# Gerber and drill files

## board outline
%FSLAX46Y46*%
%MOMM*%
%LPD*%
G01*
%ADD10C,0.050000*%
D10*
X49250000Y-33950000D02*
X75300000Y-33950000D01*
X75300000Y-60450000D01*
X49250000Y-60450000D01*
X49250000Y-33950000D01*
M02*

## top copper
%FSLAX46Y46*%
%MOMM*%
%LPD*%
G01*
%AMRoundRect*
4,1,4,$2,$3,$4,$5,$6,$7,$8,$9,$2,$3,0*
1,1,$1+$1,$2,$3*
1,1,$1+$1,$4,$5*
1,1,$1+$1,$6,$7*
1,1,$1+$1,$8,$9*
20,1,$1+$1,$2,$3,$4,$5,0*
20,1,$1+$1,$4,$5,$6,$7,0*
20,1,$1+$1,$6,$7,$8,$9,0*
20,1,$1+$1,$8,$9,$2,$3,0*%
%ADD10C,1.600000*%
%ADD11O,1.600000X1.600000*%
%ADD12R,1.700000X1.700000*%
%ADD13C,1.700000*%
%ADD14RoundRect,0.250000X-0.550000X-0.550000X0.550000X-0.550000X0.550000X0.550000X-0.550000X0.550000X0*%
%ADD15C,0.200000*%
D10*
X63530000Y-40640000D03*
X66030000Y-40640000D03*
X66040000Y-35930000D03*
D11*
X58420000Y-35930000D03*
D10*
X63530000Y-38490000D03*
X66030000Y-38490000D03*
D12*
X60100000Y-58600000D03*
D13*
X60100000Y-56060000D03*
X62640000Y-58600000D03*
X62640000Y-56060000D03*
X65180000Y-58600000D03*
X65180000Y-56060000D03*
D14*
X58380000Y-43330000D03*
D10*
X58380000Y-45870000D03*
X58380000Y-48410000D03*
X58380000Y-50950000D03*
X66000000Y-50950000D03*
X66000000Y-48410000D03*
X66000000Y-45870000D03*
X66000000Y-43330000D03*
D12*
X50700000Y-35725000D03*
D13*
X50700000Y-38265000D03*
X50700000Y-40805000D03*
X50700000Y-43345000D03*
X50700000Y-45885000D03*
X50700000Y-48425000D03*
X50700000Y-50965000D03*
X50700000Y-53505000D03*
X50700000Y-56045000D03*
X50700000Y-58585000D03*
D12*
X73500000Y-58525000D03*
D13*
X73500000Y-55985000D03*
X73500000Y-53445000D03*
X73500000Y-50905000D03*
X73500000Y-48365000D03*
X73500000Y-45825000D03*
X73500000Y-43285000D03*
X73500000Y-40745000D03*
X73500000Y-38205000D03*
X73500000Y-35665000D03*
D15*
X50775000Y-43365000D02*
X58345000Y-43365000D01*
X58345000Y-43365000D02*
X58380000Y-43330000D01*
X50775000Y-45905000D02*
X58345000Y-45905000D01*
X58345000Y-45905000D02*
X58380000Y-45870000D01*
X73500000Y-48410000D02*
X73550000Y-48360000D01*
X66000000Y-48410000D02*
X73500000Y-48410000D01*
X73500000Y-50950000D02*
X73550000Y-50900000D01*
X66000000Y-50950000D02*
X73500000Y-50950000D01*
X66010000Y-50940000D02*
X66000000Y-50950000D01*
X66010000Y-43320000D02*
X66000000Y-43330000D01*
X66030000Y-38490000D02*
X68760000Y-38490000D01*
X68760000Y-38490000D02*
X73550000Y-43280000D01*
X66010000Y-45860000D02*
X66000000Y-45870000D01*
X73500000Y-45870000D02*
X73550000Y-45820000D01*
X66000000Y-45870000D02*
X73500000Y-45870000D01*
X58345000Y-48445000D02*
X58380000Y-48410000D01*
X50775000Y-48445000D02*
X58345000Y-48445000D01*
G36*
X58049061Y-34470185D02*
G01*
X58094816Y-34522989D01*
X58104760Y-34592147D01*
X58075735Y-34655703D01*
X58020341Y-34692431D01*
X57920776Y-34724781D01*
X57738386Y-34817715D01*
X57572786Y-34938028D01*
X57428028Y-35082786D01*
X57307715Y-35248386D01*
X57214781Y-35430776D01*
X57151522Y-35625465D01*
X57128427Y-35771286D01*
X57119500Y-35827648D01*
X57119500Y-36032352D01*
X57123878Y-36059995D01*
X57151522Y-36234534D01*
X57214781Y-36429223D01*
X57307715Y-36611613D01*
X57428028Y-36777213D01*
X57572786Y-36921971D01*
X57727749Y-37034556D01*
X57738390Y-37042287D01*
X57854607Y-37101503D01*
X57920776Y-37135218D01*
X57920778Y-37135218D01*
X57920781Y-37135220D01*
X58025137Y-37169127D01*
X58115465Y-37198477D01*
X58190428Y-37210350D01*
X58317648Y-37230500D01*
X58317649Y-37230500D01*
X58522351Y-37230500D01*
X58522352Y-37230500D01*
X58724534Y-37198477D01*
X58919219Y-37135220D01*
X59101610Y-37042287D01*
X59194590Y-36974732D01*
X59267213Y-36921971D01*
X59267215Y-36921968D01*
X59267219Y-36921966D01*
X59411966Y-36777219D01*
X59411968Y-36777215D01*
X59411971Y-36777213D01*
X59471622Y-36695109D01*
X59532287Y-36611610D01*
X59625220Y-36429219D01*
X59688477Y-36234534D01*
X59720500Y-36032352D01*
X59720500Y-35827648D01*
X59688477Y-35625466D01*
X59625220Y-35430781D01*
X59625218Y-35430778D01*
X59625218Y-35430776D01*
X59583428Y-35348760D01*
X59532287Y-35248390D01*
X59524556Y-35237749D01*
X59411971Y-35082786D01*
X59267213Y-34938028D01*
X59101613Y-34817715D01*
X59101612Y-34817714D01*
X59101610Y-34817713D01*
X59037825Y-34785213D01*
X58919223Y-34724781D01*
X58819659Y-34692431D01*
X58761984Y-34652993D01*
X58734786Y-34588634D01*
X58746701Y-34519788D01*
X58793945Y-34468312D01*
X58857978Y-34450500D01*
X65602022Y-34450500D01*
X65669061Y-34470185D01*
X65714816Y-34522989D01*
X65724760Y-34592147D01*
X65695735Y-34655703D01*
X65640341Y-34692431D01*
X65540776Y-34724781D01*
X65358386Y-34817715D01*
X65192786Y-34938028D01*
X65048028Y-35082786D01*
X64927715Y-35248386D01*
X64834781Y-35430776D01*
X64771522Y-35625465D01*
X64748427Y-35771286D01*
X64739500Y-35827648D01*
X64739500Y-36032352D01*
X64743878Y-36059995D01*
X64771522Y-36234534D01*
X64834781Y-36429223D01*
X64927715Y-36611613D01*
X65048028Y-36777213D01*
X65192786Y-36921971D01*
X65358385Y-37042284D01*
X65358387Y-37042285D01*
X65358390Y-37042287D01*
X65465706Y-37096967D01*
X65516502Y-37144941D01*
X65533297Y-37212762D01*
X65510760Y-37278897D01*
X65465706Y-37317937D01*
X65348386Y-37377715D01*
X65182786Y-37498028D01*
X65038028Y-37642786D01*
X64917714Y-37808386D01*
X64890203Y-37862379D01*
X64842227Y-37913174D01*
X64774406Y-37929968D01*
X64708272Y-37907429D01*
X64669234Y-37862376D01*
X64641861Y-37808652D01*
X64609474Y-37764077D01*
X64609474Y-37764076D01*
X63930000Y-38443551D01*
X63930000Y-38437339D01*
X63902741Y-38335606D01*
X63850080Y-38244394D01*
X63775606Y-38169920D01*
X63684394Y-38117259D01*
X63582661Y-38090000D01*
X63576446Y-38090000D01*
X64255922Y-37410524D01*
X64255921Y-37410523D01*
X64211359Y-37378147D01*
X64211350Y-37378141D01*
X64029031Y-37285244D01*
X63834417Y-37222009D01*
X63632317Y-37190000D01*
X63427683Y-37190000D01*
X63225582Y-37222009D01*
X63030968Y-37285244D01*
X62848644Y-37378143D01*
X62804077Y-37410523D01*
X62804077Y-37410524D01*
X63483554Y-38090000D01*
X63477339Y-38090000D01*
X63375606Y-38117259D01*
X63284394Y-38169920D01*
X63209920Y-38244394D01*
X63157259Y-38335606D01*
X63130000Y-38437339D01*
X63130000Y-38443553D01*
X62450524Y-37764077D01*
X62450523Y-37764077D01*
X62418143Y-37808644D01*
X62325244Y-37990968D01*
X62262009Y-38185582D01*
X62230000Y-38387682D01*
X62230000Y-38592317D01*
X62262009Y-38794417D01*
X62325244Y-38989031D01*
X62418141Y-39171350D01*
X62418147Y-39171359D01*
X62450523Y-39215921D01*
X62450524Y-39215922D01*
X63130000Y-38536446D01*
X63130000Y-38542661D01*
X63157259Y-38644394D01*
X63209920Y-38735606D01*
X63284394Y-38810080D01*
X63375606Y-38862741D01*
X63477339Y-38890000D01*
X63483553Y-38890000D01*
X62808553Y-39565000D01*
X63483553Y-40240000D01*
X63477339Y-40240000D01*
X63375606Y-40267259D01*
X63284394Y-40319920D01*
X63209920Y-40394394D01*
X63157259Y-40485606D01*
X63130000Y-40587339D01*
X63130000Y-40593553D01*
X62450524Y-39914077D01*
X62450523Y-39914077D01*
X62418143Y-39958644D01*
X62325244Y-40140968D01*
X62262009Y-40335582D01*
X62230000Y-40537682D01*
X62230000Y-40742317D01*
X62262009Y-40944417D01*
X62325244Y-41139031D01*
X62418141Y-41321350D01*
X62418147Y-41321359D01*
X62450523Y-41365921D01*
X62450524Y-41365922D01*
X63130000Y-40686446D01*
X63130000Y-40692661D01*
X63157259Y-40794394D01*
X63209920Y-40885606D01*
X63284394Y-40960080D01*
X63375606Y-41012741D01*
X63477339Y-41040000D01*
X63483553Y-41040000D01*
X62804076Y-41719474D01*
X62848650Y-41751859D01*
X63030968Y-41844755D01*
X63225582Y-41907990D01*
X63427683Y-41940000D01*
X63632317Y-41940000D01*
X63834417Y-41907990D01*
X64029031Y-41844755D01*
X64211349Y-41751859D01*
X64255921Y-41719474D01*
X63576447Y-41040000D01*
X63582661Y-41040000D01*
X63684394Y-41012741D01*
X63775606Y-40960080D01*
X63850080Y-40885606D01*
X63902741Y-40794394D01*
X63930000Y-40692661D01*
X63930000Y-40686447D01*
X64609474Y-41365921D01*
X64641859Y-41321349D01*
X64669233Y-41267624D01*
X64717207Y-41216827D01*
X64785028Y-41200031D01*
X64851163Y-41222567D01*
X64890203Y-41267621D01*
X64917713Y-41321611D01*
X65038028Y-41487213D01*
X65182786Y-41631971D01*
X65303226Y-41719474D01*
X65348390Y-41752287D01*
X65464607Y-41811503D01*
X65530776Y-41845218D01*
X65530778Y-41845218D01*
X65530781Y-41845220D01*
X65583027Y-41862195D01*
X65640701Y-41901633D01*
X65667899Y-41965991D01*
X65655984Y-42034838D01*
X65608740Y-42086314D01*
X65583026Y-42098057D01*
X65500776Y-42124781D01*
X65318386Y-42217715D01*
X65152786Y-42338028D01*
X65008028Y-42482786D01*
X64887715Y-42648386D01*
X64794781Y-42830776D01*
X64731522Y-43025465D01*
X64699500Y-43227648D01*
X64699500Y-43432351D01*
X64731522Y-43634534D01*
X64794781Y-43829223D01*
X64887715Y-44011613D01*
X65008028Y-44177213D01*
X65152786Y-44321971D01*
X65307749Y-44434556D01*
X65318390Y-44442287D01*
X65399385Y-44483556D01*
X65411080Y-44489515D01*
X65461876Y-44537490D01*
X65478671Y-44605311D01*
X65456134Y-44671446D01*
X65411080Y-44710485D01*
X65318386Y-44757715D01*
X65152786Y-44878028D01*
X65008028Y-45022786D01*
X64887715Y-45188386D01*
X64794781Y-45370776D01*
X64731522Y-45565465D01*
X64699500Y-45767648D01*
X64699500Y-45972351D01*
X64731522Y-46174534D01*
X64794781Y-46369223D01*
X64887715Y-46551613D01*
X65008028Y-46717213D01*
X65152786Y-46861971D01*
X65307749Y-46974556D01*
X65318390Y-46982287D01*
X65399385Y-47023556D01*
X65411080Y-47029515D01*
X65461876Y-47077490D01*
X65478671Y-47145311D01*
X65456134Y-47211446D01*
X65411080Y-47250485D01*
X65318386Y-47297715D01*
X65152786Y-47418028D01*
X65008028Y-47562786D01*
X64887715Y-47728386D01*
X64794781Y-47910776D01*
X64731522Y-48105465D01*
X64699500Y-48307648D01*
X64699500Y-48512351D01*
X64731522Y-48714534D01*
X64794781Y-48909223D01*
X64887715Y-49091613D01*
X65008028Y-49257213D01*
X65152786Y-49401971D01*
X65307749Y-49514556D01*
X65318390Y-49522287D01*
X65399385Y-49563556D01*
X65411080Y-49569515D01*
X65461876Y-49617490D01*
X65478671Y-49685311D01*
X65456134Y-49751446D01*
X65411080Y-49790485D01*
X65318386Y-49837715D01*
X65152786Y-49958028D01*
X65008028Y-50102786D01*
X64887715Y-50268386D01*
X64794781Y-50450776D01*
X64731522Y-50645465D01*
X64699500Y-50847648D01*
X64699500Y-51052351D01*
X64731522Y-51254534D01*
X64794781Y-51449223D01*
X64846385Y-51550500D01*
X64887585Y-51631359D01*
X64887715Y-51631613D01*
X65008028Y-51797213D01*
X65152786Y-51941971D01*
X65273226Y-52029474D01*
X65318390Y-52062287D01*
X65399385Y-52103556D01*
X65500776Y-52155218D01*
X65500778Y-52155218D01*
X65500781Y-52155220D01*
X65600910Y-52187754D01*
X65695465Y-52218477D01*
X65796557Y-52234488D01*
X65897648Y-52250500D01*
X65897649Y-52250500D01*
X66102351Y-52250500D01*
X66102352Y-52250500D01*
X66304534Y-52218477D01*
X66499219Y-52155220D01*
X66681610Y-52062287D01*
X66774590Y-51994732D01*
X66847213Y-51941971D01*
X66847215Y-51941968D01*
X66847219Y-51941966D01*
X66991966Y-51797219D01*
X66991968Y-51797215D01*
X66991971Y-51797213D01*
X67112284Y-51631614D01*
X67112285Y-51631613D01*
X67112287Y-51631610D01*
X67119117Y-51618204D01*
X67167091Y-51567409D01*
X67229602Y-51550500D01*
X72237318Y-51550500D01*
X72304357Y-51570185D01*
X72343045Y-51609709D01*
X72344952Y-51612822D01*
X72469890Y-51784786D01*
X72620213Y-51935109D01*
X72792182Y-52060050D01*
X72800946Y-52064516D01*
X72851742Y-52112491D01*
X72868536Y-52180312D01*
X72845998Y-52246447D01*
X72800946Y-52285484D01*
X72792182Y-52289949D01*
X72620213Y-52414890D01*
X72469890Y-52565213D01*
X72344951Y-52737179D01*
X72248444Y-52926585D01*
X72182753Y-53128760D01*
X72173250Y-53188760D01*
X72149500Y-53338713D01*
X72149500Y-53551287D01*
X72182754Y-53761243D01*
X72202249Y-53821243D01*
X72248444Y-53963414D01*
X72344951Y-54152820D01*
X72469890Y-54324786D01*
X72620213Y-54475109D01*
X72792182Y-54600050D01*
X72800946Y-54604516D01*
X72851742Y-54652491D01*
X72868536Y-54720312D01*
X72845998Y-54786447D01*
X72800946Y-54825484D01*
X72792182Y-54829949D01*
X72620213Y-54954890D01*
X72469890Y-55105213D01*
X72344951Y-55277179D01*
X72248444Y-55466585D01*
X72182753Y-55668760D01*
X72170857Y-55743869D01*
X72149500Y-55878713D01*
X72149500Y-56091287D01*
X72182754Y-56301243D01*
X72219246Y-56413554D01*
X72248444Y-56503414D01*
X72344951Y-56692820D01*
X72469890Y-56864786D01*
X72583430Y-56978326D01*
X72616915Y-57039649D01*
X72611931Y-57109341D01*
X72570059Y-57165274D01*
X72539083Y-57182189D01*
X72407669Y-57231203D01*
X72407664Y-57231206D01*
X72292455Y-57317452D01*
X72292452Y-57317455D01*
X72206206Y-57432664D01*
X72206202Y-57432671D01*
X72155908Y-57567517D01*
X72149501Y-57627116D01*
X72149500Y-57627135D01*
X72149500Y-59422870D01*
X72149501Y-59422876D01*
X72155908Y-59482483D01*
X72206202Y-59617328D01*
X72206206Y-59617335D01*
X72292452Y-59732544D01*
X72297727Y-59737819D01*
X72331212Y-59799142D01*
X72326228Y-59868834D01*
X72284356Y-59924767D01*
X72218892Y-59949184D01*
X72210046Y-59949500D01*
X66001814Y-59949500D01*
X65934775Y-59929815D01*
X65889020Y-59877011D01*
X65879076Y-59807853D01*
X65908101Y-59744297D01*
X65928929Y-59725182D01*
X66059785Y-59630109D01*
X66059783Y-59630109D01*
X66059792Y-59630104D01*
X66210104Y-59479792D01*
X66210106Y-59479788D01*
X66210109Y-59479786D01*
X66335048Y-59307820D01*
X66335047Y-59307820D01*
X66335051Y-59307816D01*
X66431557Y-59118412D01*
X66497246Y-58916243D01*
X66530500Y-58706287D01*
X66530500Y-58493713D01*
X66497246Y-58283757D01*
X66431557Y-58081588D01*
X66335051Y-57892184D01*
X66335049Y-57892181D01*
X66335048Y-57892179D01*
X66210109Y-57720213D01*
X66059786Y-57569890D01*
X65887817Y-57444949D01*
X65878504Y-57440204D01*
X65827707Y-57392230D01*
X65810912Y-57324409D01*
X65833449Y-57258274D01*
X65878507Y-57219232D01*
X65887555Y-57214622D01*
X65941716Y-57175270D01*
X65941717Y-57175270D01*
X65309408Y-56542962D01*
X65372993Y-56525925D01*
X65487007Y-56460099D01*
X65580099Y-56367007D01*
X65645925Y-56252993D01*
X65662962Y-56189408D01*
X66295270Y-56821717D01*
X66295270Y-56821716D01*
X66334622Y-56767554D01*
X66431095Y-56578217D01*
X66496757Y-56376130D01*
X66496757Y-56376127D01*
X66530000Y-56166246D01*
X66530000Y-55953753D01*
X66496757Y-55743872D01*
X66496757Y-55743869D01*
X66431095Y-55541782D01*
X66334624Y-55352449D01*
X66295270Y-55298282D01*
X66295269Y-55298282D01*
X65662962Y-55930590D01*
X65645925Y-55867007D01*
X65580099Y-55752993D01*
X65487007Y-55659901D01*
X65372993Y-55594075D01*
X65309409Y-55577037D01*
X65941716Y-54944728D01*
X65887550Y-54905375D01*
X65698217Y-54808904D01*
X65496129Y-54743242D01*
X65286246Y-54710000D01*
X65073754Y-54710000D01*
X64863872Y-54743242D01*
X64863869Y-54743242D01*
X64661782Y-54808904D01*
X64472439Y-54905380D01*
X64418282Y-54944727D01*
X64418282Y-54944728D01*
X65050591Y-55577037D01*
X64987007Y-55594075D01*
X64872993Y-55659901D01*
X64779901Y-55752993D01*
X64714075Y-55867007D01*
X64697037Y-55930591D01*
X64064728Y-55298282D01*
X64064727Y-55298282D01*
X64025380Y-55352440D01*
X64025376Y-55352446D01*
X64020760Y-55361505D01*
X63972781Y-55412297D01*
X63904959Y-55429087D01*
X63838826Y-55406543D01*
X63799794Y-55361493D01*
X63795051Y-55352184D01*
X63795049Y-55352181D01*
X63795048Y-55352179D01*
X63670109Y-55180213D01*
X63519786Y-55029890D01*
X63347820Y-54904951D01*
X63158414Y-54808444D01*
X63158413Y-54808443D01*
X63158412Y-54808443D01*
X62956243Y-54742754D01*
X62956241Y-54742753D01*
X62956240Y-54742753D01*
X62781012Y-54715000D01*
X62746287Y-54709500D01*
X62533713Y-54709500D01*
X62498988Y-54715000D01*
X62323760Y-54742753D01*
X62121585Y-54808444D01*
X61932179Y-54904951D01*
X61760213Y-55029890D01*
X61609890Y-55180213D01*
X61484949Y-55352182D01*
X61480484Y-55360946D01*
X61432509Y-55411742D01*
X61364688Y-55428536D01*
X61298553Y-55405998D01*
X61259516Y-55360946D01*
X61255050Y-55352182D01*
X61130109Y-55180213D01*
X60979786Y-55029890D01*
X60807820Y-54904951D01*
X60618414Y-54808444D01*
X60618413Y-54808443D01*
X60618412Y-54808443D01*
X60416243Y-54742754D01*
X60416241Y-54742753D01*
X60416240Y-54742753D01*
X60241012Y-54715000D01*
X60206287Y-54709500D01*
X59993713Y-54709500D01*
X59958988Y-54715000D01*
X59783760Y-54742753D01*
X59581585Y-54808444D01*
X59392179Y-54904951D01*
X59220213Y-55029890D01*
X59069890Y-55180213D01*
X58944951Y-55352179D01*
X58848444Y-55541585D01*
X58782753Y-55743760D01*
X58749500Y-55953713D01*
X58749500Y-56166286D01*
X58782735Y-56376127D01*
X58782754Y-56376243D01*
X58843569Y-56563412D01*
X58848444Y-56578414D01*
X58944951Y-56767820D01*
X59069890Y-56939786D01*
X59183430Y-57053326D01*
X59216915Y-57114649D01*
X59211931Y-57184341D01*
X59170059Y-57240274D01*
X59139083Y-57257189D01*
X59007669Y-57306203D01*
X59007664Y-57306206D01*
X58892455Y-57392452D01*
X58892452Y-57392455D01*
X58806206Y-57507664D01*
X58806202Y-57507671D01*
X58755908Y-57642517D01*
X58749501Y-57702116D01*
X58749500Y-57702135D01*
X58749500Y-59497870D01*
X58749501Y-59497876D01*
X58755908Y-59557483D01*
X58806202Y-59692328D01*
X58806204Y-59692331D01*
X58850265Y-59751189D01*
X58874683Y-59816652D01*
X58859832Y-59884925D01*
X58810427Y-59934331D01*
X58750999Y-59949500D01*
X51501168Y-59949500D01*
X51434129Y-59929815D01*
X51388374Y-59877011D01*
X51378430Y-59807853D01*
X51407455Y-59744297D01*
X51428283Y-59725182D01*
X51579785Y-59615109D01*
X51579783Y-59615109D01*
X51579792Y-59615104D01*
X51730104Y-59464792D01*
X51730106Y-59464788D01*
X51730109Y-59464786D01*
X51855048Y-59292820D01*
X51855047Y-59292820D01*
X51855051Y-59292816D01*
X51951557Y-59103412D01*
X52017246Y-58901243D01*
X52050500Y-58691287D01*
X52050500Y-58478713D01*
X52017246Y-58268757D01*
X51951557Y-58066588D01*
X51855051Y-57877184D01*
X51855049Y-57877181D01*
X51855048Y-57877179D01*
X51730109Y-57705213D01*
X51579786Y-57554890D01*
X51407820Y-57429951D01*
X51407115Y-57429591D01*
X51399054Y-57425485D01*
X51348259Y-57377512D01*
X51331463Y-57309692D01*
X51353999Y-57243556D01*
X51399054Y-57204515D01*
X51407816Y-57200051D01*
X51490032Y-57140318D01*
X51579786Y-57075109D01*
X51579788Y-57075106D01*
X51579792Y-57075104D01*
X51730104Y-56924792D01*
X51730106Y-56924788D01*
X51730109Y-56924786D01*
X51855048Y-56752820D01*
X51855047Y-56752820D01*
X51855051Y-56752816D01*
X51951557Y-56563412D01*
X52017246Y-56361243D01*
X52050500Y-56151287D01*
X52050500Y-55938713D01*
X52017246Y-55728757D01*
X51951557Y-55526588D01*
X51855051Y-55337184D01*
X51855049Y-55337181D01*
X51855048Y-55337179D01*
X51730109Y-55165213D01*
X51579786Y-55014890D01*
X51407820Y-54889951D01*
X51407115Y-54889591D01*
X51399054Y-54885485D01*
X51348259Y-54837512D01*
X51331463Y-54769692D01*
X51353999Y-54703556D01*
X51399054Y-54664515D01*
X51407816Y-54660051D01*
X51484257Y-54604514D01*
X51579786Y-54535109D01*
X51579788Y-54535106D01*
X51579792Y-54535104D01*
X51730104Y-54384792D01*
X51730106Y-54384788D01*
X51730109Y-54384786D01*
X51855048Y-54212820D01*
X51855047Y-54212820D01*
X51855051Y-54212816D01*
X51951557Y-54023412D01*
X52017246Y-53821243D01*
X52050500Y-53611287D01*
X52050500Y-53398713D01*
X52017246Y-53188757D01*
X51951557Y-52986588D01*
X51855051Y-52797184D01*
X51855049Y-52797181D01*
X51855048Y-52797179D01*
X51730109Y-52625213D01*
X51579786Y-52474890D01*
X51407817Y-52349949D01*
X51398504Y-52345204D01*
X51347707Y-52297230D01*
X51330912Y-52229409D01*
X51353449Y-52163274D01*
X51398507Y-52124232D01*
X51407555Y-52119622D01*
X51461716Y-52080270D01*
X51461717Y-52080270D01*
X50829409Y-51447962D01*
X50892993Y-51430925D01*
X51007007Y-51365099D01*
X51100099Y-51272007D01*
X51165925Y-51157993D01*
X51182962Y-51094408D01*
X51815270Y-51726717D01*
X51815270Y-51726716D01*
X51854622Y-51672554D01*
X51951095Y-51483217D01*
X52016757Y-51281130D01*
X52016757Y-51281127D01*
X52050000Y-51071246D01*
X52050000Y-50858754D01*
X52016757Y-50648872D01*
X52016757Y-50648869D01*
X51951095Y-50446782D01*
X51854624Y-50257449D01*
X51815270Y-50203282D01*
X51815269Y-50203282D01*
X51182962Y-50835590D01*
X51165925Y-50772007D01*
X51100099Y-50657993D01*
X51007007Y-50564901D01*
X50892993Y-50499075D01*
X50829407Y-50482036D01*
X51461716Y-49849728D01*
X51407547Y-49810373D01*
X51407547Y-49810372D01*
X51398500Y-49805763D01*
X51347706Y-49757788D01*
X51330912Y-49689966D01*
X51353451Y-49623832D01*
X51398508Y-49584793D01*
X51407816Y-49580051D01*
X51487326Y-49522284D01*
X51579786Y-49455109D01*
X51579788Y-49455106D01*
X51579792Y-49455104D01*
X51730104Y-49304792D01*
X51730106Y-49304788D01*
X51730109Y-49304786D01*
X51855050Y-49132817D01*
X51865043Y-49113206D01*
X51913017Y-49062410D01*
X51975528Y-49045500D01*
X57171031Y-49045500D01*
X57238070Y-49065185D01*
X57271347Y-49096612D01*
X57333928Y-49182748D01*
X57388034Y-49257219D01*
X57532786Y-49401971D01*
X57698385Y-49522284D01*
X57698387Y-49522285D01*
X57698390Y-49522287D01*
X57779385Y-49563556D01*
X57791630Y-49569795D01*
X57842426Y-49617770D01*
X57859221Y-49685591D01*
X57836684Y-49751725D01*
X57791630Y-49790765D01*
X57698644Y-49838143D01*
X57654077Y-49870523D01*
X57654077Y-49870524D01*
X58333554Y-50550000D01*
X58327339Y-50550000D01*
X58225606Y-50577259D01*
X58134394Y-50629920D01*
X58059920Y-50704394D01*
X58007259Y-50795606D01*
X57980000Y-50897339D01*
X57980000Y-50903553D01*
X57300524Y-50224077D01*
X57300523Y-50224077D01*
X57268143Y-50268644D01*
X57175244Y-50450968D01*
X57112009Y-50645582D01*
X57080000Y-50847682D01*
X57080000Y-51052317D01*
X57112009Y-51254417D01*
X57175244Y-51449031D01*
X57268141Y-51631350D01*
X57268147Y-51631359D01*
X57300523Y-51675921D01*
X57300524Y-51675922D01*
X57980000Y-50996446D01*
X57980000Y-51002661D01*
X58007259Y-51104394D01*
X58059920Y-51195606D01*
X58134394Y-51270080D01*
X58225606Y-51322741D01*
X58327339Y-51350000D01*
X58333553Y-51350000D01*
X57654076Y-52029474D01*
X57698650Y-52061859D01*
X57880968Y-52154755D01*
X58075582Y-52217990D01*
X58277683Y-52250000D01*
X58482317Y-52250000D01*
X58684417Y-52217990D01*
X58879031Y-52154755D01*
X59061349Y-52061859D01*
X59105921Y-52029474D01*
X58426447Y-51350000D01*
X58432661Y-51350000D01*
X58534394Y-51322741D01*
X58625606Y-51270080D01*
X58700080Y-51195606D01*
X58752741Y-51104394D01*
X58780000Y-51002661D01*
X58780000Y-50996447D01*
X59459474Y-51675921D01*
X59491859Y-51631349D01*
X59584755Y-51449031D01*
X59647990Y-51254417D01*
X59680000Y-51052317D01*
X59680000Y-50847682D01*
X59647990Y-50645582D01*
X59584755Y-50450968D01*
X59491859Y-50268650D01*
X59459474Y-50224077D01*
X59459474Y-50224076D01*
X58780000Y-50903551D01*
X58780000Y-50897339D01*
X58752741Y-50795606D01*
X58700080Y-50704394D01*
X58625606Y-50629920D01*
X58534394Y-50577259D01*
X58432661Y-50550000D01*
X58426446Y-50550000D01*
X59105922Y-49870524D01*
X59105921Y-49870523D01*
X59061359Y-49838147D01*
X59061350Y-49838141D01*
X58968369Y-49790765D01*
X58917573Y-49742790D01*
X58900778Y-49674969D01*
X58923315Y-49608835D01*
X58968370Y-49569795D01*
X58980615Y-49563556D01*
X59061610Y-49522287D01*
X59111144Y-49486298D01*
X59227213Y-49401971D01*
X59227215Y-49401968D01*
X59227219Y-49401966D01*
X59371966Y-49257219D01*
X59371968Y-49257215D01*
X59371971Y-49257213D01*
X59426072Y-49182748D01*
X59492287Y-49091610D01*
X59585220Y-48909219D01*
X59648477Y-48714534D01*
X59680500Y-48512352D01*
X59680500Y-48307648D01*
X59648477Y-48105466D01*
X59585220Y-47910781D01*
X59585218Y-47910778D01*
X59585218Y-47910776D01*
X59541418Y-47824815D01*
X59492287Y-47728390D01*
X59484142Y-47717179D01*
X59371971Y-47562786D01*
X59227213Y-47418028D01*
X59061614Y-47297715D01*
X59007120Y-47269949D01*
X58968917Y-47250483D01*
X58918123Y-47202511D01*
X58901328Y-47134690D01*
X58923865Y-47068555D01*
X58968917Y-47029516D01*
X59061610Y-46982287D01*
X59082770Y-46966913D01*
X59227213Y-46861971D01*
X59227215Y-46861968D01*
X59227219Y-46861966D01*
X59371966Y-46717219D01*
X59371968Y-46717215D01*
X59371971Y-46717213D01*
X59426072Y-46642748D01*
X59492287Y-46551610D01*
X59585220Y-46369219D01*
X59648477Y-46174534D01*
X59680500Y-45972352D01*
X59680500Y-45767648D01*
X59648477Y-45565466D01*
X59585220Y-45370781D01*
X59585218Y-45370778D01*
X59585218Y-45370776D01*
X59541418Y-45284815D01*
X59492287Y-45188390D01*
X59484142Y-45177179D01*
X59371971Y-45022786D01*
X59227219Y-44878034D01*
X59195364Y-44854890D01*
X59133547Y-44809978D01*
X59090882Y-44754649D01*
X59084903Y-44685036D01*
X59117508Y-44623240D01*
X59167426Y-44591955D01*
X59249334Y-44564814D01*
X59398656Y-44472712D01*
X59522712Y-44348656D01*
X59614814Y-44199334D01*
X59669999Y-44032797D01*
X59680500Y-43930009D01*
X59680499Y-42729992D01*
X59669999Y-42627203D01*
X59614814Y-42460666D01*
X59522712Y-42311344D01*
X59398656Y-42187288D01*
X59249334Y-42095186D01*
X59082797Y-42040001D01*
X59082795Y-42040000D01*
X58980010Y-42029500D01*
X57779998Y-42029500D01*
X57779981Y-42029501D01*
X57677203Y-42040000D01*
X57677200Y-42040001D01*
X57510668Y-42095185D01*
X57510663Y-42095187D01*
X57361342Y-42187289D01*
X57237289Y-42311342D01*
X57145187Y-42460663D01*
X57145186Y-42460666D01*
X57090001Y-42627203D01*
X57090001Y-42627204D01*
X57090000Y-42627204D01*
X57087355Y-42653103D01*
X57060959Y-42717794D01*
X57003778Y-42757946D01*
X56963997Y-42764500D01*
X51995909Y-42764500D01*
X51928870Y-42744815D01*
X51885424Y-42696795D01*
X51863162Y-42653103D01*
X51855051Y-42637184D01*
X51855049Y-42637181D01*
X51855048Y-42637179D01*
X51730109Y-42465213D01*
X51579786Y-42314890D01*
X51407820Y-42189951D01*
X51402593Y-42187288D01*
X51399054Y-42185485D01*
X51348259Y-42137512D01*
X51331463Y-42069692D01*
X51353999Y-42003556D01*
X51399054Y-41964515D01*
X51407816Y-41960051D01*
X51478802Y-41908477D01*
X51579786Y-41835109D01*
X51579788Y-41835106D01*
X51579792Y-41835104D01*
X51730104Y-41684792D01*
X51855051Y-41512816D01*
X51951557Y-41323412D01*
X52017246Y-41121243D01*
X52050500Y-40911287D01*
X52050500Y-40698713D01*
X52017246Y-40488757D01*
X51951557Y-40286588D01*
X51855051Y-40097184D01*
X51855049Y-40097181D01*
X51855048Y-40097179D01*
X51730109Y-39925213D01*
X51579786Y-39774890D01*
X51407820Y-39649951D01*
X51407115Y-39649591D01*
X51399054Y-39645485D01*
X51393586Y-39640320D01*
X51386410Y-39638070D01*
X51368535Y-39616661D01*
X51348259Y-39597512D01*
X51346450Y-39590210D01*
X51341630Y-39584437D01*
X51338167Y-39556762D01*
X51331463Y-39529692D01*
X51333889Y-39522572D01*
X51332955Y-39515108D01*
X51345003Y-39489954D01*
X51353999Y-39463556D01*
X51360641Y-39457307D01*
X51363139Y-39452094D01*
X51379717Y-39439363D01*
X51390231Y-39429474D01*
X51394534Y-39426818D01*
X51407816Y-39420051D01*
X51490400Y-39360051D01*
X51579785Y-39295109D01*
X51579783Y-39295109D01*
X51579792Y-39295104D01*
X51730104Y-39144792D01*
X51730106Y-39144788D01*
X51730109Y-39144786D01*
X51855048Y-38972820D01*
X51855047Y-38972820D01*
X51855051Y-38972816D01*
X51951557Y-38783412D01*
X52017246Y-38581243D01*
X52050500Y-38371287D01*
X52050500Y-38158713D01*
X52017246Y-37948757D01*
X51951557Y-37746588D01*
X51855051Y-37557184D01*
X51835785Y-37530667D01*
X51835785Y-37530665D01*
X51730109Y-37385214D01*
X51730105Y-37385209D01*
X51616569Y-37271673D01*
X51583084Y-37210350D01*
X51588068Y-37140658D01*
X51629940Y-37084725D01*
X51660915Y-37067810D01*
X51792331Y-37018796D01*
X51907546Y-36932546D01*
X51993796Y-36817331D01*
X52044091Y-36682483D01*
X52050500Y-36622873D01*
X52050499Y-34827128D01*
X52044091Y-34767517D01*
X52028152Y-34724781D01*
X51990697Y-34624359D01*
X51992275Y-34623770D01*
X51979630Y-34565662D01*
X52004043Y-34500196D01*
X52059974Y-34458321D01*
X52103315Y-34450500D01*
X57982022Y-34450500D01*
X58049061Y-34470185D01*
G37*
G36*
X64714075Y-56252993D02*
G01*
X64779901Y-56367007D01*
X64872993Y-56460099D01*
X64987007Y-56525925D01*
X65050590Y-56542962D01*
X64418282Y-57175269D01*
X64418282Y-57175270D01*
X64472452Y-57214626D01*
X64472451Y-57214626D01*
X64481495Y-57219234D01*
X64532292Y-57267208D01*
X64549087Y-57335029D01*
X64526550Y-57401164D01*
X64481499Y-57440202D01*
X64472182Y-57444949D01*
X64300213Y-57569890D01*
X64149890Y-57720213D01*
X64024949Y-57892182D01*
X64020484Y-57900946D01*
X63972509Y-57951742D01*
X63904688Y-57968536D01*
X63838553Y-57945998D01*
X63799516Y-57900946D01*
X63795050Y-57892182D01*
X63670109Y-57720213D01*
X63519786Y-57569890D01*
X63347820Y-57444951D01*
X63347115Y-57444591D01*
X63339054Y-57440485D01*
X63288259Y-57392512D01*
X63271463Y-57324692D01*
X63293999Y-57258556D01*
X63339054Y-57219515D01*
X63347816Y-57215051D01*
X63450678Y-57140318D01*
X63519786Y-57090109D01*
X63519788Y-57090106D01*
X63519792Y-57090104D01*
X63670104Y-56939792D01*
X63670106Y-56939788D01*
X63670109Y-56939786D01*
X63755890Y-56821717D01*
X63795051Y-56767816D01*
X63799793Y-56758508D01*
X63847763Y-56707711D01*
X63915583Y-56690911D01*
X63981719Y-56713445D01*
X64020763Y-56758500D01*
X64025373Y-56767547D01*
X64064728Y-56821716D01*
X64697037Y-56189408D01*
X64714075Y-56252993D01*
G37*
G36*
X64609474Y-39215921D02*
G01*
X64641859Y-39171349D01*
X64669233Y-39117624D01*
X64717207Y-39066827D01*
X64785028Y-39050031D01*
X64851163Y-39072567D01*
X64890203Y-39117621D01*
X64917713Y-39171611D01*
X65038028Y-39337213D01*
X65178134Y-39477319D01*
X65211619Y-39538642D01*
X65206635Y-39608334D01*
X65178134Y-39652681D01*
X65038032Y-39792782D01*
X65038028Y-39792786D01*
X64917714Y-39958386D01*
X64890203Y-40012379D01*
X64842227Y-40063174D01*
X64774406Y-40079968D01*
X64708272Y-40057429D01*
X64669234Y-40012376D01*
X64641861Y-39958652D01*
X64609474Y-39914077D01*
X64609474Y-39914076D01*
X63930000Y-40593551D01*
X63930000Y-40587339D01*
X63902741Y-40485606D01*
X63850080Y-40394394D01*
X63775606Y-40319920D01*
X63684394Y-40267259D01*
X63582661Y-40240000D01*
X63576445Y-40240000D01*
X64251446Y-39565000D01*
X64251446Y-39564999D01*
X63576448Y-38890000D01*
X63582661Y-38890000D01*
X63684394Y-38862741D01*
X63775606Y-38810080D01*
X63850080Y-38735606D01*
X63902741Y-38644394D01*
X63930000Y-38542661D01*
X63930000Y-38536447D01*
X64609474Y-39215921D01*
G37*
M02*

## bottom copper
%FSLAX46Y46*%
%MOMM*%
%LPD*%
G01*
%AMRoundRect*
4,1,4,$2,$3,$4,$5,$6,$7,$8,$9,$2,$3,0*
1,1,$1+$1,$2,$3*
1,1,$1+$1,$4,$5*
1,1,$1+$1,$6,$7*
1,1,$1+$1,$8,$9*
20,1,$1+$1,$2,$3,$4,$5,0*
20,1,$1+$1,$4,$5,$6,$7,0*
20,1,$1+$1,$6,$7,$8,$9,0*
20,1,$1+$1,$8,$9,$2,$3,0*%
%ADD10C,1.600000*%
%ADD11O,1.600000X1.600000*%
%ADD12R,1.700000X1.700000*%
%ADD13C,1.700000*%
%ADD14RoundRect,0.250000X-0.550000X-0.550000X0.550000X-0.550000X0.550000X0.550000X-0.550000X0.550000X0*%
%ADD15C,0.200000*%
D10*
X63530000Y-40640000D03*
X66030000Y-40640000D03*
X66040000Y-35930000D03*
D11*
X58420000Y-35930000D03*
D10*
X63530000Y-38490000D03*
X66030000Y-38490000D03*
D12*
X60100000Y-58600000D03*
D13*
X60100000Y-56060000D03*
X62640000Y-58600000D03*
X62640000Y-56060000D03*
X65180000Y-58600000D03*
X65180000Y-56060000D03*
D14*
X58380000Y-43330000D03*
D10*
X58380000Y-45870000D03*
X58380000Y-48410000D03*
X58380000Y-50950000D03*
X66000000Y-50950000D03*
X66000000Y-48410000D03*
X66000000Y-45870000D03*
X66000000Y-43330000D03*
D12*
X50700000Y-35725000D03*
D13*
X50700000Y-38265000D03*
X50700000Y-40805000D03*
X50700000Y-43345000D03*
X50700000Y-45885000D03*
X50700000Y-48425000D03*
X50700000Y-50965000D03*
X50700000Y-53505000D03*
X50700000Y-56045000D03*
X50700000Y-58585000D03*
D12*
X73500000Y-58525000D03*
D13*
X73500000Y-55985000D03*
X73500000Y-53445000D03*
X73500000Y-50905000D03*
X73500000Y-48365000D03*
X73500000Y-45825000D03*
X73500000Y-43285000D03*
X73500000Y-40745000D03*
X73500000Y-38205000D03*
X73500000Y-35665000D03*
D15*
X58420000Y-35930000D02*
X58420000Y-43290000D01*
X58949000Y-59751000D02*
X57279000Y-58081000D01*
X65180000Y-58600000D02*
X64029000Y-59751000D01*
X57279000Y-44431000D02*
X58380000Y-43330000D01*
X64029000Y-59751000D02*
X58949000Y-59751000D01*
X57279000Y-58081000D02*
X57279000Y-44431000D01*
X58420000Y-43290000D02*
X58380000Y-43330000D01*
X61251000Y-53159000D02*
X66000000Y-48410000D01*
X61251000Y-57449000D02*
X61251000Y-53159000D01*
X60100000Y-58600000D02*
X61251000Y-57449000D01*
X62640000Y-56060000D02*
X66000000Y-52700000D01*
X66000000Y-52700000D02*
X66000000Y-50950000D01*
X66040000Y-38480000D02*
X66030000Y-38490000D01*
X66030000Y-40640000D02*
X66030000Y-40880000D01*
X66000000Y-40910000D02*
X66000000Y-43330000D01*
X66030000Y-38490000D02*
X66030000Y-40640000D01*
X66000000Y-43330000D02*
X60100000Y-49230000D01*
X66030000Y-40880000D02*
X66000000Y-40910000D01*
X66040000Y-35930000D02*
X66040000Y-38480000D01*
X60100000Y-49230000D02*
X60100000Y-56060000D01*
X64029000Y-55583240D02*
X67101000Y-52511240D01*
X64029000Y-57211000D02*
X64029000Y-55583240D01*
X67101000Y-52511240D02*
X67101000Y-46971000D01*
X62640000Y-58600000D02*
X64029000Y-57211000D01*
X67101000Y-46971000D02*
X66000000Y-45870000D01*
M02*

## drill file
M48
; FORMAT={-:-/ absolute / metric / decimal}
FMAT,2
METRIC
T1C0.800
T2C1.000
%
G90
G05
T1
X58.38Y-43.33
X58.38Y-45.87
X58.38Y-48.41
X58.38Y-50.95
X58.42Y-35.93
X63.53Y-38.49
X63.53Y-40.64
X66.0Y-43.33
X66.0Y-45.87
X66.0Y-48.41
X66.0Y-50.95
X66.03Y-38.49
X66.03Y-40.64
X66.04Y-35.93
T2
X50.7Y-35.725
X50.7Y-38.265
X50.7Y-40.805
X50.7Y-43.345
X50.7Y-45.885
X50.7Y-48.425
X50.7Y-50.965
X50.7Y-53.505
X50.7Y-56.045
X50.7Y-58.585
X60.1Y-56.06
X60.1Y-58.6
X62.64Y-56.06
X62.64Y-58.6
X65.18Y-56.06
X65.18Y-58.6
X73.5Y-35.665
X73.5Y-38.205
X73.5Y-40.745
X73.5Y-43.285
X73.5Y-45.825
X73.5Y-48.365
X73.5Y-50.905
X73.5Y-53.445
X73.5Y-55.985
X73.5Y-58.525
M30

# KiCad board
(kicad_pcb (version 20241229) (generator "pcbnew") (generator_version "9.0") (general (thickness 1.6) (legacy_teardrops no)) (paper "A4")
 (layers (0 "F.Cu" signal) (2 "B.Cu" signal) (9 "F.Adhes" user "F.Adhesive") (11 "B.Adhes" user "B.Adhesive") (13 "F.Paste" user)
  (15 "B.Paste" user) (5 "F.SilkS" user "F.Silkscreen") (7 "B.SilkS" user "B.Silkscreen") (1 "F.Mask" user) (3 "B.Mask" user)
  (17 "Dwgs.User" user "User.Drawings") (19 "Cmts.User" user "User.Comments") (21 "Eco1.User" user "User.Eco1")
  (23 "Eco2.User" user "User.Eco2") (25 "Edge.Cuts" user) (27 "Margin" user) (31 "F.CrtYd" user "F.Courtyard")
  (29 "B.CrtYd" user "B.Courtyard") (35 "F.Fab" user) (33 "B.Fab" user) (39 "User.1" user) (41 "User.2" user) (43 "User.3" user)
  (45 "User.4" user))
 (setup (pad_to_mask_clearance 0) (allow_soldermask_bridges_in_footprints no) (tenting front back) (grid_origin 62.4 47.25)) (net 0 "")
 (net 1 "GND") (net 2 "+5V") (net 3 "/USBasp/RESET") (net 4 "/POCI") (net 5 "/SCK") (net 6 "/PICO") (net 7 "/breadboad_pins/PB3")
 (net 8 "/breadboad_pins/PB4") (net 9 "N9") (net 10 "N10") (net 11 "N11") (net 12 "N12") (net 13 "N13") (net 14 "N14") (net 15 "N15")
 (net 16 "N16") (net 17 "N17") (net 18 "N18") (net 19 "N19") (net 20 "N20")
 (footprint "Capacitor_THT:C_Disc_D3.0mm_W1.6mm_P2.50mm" (layer "F.Cu") (at 63.53 40.64)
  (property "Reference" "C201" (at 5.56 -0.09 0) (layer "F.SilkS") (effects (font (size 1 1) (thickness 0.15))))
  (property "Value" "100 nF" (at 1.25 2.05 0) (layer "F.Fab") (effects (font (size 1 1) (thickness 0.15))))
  (pad "1" thru_hole circle (at 0 0) (size 1.6 1.6) (drill 0.8) (layers "*.Cu" "*.Mask") (remove_unused_layers no) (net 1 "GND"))
  (pad "2" thru_hole circle (at 2.5 0) (size 1.6 1.6) (drill 0.8) (layers "*.Cu" "*.Mask") (remove_unused_layers no) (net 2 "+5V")))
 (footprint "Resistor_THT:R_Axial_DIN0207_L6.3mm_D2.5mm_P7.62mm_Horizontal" (layer "F.Cu") (at 66.04 35.93 180)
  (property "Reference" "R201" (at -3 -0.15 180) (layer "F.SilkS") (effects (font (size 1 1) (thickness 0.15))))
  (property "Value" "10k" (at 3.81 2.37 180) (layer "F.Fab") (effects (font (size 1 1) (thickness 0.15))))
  (pad "1" thru_hole circle (at 0 0 180) (size 1.6 1.6) (drill 0.8) (layers "*.Cu" "*.Mask") (remove_unused_layers no) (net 2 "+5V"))
  (pad "2" thru_hole oval (at 7.62 0 180) (size 1.6 1.6) (drill 0.8) (layers "*.Cu" "*.Mask") (remove_unused_layers no)
   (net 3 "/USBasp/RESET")))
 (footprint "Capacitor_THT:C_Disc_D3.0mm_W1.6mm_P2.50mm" (layer "F.Cu") (at 63.53 38.49)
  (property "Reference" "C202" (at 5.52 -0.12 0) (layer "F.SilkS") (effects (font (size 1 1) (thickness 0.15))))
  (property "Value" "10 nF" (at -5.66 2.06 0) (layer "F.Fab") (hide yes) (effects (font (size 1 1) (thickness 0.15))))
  (pad "1" thru_hole circle (at 0 0) (size 1.6 1.6) (drill 0.8) (layers "*.Cu" "*.Mask") (remove_unused_layers no) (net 1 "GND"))
  (pad "2" thru_hole circle (at 2.5 0) (size 1.6 1.6) (drill 0.8) (layers "*.Cu" "*.Mask") (remove_unused_layers no) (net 2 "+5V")))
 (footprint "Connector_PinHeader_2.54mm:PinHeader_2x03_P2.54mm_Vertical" (layer "F.Cu") (at 60.1 58.6 90)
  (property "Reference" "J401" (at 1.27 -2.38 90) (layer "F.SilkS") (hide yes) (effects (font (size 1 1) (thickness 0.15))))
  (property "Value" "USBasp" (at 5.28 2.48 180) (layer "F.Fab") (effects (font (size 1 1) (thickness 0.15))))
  (pad "1" thru_hole rect (at 0 0 90) (size 1.7 1.7) (drill 1) (layers "*.Cu" "*.Mask") (remove_unused_layers no) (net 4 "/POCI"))
  (pad "2" thru_hole circle (at 2.54 0 90) (size 1.7 1.7) (drill 1) (layers "*.Cu" "*.Mask") (remove_unused_layers no) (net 2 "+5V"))
  (pad "3" thru_hole circle (at 0 2.54 90) (size 1.7 1.7) (drill 1) (layers "*.Cu" "*.Mask") (remove_unused_layers no) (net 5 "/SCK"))
  (pad "4" thru_hole circle (at 2.54 2.54 90) (size 1.7 1.7) (drill 1) (layers "*.Cu" "*.Mask") (remove_unused_layers no) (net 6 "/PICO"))
  (pad "5" thru_hole circle (at 0 5.08 90) (size 1.7 1.7) (drill 1) (layers "*.Cu" "*.Mask") (remove_unused_layers no)
   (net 3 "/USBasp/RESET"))
  (pad "6" thru_hole circle (at 2.54 5.08 90) (size 1.7 1.7) (drill 1) (layers "*.Cu" "*.Mask") (remove_unused_layers no) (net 1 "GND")))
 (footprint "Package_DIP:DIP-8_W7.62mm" (layer "F.Cu") (at 58.38 43.33)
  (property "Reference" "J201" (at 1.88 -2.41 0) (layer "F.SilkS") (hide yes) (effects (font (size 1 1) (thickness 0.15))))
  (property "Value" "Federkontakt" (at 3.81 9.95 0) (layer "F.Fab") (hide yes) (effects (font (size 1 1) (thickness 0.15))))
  (pad "1" thru_hole roundrect (at 0 0) (size 1.6 1.6) (drill 0.8) (layers "*.Cu" "*.Mask") (remove_unused_layers no)
   (roundrect_rratio 0.15625) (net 3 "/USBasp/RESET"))
  (pad "2" thru_hole circle (at 0 2.54) (size 1.6 1.6) (drill 0.8) (layers "*.Cu" "*.Mask") (remove_unused_layers no)
   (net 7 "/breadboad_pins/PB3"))
  (pad "3" thru_hole circle (at 0 5.08) (size 1.6 1.6) (drill 0.8) (layers "*.Cu" "*.Mask") (remove_unused_layers no)
   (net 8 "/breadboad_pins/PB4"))
  (pad "4" thru_hole circle (at 0 7.62) (size 1.6 1.6) (drill 0.8) (layers "*.Cu" "*.Mask") (remove_unused_layers no) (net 1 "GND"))
  (pad "5" thru_hole circle (at 7.62 7.62) (size 1.6 1.6) (drill 0.8) (layers "*.Cu" "*.Mask") (remove_unused_layers no) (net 6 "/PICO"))
  (pad "6" thru_hole circle (at 7.62 5.08) (size 1.6 1.6) (drill 0.8) (layers "*.Cu" "*.Mask") (remove_unused_layers no) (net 4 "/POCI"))
  (pad "7" thru_hole circle (at 7.62 2.54) (size 1.6 1.6) (drill 0.8) (layers "*.Cu" "*.Mask") (remove_unused_layers no) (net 5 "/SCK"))
  (pad "8" thru_hole circle (at 7.62 0) (size 1.6 1.6) (drill 0.8) (layers "*.Cu" "*.Mask") (remove_unused_layers no) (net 2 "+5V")))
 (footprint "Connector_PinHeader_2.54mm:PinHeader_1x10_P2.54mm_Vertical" (layer "B.Cu") (at 50.7 35.725 180)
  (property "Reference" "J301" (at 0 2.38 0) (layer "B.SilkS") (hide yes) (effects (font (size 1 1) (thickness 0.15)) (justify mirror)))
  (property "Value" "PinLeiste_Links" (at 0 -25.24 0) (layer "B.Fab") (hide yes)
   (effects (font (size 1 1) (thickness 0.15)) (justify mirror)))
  (pad "1" thru_hole rect (at 0 0 180) (size 1.7 1.7) (drill 1) (layers "*.Cu" "*.Mask") (remove_unused_layers no) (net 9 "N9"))
  (pad "2" thru_hole circle (at 0 -2.54 180) (size 1.7 1.7) (drill 1) (layers "*.Cu" "*.Mask") (remove_unused_layers no) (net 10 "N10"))
  (pad "3" thru_hole circle (at 0 -5.08 180) (size 1.7 1.7) (drill 1) (layers "*.Cu" "*.Mask") (remove_unused_layers no) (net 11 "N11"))
  (pad "4" thru_hole circle (at 0 -7.62 180) (size 1.7 1.7) (drill 1) (layers "*.Cu" "*.Mask") (remove_unused_layers no)
   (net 3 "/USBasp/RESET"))
  (pad "5" thru_hole circle (at 0 -10.16 180) (size 1.7 1.7) (drill 1) (layers "*.Cu" "*.Mask") (remove_unused_layers no)
   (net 7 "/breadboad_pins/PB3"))
  (pad "6" thru_hole circle (at 0 -12.7 180) (size 1.7 1.7) (drill 1) (layers "*.Cu" "*.Mask") (remove_unused_layers no)
   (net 8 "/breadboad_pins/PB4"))
  (pad "7" thru_hole circle (at 0 -15.24 180) (size 1.7 1.7) (drill 1) (layers "*.Cu" "*.Mask") (remove_unused_layers no) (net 1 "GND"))
  (pad "8" thru_hole circle (at 0 -17.78 180) (size 1.7 1.7) (drill 1) (layers "*.Cu" "*.Mask") (remove_unused_layers no) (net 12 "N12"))
  (pad "9" thru_hole circle (at 0 -20.32 180) (size 1.7 1.7) (drill 1) (layers "*.Cu" "*.Mask") (remove_unused_layers no) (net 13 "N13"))
  (pad "10" thru_hole circle (at 0 -22.86 180) (size 1.7 1.7) (drill 1) (layers "*.Cu" "*.Mask") (remove_unused_layers no) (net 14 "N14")))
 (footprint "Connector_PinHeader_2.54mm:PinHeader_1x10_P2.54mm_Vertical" (layer "B.Cu") (at 73.5 58.525)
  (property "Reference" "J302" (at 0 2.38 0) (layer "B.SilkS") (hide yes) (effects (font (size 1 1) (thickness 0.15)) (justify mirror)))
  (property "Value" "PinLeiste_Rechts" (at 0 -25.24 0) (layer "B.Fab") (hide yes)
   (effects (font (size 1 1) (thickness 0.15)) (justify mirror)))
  (pad "1" thru_hole rect (at 0 0) (size 1.7 1.7) (drill 1) (layers "*.Cu" "*.Mask") (remove_unused_layers no) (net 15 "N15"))
  (pad "2" thru_hole circle (at 0 -2.54) (size 1.7 1.7) (drill 1) (layers "*.Cu" "*.Mask") (remove_unused_layers no) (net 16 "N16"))
  (pad "3" thru_hole circle (at 0 -5.08) (size 1.7 1.7) (drill 1) (layers "*.Cu" "*.Mask") (remove_unused_layers no) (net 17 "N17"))
  (pad "4" thru_hole circle (at 0 -7.62) (size 1.7 1.7) (drill 1) (layers "*.Cu" "*.Mask") (remove_unused_layers no) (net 6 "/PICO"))
  (pad "5" thru_hole circle (at 0 -10.16) (size 1.7 1.7) (drill 1) (layers "*.Cu" "*.Mask") (remove_unused_layers no) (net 4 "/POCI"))
  (pad "6" thru_hole circle (at 0 -12.7) (size 1.7 1.7) (drill 1) (layers "*.Cu" "*.Mask") (remove_unused_layers no) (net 5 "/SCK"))
  (pad "7" thru_hole circle (at 0 -15.24) (size 1.7 1.7) (drill 1) (layers "*.Cu" "*.Mask") (remove_unused_layers no) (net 2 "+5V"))
  (pad "8" thru_hole circle (at 0 -17.78) (size 1.7 1.7) (drill 1) (layers "*.Cu" "*.Mask") (remove_unused_layers no) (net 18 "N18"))
  (pad "9" thru_hole circle (at 0 -20.32) (size 1.7 1.7) (drill 1) (layers "*.Cu" "*.Mask") (remove_unused_layers no) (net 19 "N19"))
  (pad "10" thru_hole circle (at 0 -22.86) (size 1.7 1.7) (drill 1) (layers "*.Cu" "*.Mask") (remove_unused_layers no) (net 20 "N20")))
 (gr_rect (start 49.25 33.95) (end 75.3 60.45) (stroke (width 0.05) (type solid)) (fill no) (layer "Edge.Cuts"))
 (segment (start 50.775 43.365) (end 58.345 43.365) (width 0.2) (layer "F.Cu") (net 3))
 (segment (start 58.345 43.365) (end 58.38 43.33) (width 0.2) (layer "F.Cu") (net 3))
 (segment (start 58.42 35.93) (end 58.42 43.29) (width 0.2) (layer "B.Cu") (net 3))
 (segment (start 58.949 59.751) (end 57.279 58.081) (width 0.2) (layer "B.Cu") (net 3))
 (segment (start 65.18 58.6) (end 64.029 59.751) (width 0.2) (layer "B.Cu") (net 3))
 (segment (start 57.279 44.431) (end 58.38 43.33) (width 0.2) (layer "B.Cu") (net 3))
 (segment (start 64.029 59.751) (end 58.949 59.751) (width 0.2) (layer "B.Cu") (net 3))
 (segment (start 57.279 58.081) (end 57.279 44.431) (width 0.2) (layer "B.Cu") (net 3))
 (segment (start 58.42 43.29) (end 58.38 43.33) (width 0.2) (layer "B.Cu") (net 3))
 (segment (start 50.775 45.905) (end 58.345 45.905) (width 0.2) (layer "F.Cu") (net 7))
 (segment (start 58.345 45.905) (end 58.38 45.87) (width 0.2) (layer "F.Cu") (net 7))
 (segment (start 73.5 48.41) (end 73.55 48.36) (width 0.2) (layer "F.Cu") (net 4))
 (segment (start 66 48.41) (end 73.5 48.41) (width 0.2) (layer "F.Cu") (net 4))
 (segment (start 61.251 53.159) (end 66 48.41) (width 0.2) (layer "B.Cu") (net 4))
 (segment (start 61.251 57.449) (end 61.251 53.159) (width 0.2) (layer "B.Cu") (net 4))
 (segment (start 60.1 58.6) (end 61.251 57.449) (width 0.2) (layer "B.Cu") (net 4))
 (segment (start 73.5 50.95) (end 73.55 50.9) (width 0.2) (layer "F.Cu") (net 6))
 (segment (start 66 50.95) (end 73.5 50.95) (width 0.2) (layer "F.Cu") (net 6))
 (segment (start 66.01 50.94) (end 66 50.95) (width 0.2) (layer "F.Cu") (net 6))
 (segment (start 62.64 56.06) (end 66 52.7) (width 0.2) (layer "B.Cu") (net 6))
 (segment (start 66 52.7) (end 66 50.95) (width 0.2) (layer "B.Cu") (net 6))
 (segment (start 66.01 43.32) (end 66 43.33) (width 0.2) (layer "F.Cu") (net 2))
 (segment (start 66.03 38.49) (end 68.76 38.49) (width 0.2) (layer "F.Cu") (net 2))
 (segment (start 68.76 38.49) (end 73.55 43.28) (width 0.2) (layer "F.Cu") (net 2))
 (segment (start 66.04 38.48) (end 66.03 38.49) (width 0.2) (layer "B.Cu") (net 2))
 (segment (start 66.03 40.64) (end 66.03 40.88) (width 0.2) (layer "B.Cu") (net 2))
 (segment (start 66 40.91) (end 66 43.33) (width 0.2) (layer "B.Cu") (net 2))
 (segment (start 66.03 38.49) (end 66.03 40.64) (width 0.2) (layer "B.Cu") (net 2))
 (segment (start 66 43.33) (end 60.1 49.23) (width 0.2) (layer "B.Cu") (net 2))
 (segment (start 66.03 40.88) (end 66 40.91) (width 0.2) (layer "B.Cu") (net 2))
 (segment (start 66.04 35.93) (end 66.04 38.48) (width 0.2) (layer "B.Cu") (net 2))
 (segment (start 60.1 49.23) (end 60.1 56.06) (width 0.2) (layer "B.Cu") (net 2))
 (segment (start 66.01 45.86) (end 66 45.87) (width 0.2) (layer "F.Cu") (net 5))
 (segment (start 73.5 45.87) (end 73.55 45.82) (width 0.2) (layer "F.Cu") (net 5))
 (segment (start 66 45.87) (end 73.5 45.87) (width 0.2) (layer "F.Cu") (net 5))
 (segment (start 64.029 55.58324) (end 67.101 52.51124) (width 0.2) (layer "B.Cu") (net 5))
 (segment (start 64.029 57.211) (end 64.029 55.58324) (width 0.2) (layer "B.Cu") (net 5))
 (segment (start 67.101 52.51124) (end 67.101 46.971) (width 0.2) (layer "B.Cu") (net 5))
 (segment (start 62.64 58.6) (end 64.029 57.211) (width 0.2) (layer "B.Cu") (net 5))
 (segment (start 67.101 46.971) (end 66 45.87) (width 0.2) (layer "B.Cu") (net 5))
 (segment (start 58.345 48.445) (end 58.38 48.41) (width 0.2) (layer "F.Cu") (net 8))
 (segment (start 50.775 48.445) (end 58.345 48.445) (width 0.2) (layer "F.Cu") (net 8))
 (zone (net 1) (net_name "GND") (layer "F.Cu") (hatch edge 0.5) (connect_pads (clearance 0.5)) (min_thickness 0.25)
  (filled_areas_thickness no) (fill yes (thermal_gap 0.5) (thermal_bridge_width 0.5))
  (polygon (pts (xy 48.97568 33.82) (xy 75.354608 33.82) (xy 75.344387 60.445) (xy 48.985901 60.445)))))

